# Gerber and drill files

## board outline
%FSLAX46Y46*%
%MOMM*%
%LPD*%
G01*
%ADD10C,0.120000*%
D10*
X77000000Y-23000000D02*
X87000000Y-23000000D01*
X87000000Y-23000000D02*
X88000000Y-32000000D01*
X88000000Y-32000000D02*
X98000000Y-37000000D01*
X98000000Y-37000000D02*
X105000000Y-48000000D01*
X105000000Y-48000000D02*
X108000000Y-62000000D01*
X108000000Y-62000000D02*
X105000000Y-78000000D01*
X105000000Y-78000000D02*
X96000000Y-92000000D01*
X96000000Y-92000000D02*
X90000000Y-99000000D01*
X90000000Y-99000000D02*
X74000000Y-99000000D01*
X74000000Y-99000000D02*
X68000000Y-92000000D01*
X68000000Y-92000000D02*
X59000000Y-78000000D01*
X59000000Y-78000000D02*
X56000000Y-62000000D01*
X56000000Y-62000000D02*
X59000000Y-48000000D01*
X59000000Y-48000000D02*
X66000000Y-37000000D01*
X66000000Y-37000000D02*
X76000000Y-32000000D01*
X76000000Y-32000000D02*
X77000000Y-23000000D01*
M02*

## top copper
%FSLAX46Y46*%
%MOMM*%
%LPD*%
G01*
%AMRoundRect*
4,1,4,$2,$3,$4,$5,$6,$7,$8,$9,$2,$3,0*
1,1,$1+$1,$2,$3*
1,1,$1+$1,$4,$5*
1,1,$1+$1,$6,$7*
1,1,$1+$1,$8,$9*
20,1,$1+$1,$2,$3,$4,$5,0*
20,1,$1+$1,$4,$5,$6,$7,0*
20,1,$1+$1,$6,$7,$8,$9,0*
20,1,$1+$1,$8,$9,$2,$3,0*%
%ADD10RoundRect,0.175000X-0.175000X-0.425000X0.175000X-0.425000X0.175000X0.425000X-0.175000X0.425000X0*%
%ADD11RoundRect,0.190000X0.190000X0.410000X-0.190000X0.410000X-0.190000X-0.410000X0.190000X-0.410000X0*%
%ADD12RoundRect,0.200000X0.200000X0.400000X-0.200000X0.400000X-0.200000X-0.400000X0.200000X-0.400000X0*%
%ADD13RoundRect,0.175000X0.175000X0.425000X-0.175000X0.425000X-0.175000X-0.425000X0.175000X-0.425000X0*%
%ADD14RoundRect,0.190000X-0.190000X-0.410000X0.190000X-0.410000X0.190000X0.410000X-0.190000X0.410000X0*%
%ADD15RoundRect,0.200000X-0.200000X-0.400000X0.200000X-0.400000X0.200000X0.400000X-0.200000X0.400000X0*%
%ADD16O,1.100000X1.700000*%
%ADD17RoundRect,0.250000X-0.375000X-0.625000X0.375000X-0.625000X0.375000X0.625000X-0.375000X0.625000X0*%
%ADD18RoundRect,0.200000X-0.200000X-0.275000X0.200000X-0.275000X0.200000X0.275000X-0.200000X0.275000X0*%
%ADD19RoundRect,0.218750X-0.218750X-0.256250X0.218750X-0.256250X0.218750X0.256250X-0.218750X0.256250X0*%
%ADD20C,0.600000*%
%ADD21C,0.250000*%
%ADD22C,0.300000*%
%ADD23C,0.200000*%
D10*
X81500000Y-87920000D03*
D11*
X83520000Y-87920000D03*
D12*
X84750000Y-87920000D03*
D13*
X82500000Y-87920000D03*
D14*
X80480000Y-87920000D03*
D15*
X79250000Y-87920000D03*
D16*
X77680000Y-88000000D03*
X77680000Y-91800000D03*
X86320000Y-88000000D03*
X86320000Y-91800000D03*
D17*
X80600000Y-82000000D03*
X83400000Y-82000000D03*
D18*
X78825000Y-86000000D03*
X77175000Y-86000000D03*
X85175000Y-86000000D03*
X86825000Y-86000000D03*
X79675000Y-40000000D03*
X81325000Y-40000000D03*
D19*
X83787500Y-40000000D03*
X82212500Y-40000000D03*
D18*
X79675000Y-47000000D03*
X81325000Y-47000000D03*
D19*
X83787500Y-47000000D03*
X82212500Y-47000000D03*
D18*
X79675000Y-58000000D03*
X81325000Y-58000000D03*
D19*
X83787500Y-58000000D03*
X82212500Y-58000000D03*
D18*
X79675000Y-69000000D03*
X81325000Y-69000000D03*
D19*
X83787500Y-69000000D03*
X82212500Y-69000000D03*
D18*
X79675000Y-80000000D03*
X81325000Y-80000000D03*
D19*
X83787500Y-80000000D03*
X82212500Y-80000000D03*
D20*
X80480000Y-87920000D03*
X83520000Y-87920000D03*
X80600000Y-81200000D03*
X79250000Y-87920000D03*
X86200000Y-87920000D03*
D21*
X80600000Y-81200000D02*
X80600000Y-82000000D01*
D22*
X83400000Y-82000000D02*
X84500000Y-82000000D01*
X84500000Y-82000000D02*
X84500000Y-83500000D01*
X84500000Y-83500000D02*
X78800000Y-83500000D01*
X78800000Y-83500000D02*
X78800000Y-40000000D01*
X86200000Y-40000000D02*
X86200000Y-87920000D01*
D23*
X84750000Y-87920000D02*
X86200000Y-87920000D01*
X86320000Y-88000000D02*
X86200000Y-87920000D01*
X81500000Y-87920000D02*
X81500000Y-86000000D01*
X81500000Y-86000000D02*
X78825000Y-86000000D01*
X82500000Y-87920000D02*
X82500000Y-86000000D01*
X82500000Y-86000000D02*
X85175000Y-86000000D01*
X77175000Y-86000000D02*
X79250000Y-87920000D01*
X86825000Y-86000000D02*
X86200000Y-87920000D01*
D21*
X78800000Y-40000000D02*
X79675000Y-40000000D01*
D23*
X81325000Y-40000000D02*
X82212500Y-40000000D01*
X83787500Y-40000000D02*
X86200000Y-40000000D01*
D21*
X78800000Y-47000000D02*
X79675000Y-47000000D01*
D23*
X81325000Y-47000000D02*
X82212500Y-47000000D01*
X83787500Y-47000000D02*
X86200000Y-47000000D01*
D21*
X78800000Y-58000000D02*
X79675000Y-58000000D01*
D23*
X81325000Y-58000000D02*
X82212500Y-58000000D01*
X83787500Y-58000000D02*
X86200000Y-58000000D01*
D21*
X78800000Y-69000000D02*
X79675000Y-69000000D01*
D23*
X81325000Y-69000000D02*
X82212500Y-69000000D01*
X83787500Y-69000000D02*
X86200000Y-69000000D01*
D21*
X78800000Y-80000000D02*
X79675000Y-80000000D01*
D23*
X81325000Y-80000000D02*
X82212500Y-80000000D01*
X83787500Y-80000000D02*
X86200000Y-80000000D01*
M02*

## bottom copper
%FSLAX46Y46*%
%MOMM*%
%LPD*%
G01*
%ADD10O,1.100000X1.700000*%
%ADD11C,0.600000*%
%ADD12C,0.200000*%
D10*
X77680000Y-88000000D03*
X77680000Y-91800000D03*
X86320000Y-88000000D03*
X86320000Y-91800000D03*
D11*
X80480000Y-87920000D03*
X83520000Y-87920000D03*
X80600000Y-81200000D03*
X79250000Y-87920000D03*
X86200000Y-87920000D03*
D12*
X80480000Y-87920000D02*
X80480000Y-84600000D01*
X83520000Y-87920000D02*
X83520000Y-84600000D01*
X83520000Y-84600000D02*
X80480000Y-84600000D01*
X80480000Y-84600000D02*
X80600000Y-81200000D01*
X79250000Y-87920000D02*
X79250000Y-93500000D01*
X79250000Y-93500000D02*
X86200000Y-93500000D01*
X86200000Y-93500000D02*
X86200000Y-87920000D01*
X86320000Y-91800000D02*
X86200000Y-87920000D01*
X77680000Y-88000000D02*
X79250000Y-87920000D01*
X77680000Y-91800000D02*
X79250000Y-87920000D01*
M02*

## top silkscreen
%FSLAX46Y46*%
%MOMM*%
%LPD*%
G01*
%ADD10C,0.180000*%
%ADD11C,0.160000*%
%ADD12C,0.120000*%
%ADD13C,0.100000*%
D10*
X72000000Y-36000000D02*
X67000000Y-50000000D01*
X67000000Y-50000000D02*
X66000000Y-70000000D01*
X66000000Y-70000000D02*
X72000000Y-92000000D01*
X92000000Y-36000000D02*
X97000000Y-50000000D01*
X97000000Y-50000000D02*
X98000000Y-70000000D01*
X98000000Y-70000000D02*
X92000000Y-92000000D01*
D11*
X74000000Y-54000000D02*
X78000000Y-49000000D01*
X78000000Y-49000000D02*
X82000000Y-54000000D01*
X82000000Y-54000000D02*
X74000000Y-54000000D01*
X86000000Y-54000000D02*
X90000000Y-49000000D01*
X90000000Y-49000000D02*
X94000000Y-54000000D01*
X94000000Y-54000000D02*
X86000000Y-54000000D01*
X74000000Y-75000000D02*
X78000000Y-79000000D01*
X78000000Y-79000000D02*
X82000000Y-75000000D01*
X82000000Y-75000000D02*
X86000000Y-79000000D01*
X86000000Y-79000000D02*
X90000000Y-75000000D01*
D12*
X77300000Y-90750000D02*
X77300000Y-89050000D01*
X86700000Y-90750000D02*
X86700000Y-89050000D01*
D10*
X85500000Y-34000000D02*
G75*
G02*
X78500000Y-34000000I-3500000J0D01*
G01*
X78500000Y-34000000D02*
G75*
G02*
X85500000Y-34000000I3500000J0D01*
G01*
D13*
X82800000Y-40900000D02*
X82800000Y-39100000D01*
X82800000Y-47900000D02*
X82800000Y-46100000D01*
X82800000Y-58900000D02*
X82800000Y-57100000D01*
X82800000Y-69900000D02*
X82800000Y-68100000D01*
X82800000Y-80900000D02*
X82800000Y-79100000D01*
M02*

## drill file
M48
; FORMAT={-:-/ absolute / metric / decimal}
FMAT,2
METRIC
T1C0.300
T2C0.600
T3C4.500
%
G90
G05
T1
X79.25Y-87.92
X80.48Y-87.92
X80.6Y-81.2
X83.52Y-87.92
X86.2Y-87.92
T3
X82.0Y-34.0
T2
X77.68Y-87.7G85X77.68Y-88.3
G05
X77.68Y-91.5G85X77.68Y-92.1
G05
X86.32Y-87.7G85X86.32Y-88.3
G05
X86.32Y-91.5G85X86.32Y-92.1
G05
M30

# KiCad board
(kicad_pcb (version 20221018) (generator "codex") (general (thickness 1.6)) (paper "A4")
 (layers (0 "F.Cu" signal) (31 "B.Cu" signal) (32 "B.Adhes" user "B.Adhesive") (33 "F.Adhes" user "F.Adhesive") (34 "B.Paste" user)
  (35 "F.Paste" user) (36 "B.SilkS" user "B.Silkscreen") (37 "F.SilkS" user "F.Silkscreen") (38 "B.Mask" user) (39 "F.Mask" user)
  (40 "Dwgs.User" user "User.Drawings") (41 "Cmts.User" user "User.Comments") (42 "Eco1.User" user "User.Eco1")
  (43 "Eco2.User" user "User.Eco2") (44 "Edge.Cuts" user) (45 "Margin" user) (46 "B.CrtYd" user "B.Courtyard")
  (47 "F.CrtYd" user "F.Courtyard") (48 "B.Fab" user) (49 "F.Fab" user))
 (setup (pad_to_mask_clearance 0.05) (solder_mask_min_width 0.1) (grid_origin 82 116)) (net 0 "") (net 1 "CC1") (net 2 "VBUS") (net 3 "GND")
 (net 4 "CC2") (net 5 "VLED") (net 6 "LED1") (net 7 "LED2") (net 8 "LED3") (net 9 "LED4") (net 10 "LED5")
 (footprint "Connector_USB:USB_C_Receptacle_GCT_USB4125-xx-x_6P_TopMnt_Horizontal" (layer "F.Cu") (at 82 91)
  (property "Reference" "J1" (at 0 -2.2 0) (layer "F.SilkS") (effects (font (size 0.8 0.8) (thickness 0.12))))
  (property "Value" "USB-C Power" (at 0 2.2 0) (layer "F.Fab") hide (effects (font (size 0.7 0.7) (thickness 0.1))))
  (fp_line (start -4.7 -0.25) (end -4.7 -1.95) (stroke (width 0.12) (type solid)) (layer "F.SilkS"))
  (fp_line (start 4.7 -0.25) (end 4.7 -1.95) (stroke (width 0.12) (type solid)) (layer "F.SilkS"))
  (pad "A5" smd roundrect (at -0.5 -3.08) (size 0.7 1.2) (layers "F.Cu" "F.Paste" "F.Mask") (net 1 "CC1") (roundrect_rratio 0.25))
  (pad "A9" smd roundrect (at 1.52 -3.08 180) (size 0.76 1.2) (layers "F.Cu" "F.Paste" "F.Mask") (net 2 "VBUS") (roundrect_rratio 0.25))
  (pad "A12" smd roundrect (at 2.75 -3.08 180) (size 0.8 1.2) (layers "F.Cu" "F.Paste" "F.Mask") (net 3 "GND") (roundrect_rratio 0.25))
  (pad "B5" smd roundrect (at 0.5 -3.08 180) (size 0.7 1.2) (layers "F.Cu" "F.Paste" "F.Mask") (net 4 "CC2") (roundrect_rratio 0.25))
  (pad "B9" smd roundrect (at -1.52 -3.08) (size 0.76 1.2) (layers "F.Cu" "F.Paste" "F.Mask") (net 2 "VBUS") (roundrect_rratio 0.25))
  (pad "B12" smd roundrect (at -2.75 -3.08) (size 0.8 1.2) (layers "F.Cu" "F.Paste" "F.Mask") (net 3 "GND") (roundrect_rratio 0.25))
  (pad "SH" thru_hole oval (at -4.32 -3) (size 1.1 1.7) (drill oval 0.6 1.2) (layers "*.Cu" "*.Mask") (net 3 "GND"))
  (pad "SH" thru_hole oval (at -4.32 0.8) (size 1.1 1.7) (drill oval 0.6 1.2) (layers "*.Cu" "*.Mask") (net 3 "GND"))
  (pad "SH" thru_hole oval (at 4.32 -3) (size 1.1 1.7) (drill oval 0.6 1.2) (layers "*.Cu" "*.Mask") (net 3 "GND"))
  (pad "SH" thru_hole oval (at 4.32 0.8) (size 1.1 1.7) (drill oval 0.6 1.2) (layers "*.Cu" "*.Mask") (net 3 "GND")))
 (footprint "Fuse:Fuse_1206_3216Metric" (layer "F.Cu") (at 82 82)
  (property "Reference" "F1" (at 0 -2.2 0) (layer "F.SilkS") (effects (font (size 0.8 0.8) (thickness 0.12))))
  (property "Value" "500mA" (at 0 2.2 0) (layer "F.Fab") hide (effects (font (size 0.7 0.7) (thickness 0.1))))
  (pad "1" smd roundrect (at -1.4 0) (size 1.25 1.75) (layers "F.Cu" "F.Paste" "F.Mask") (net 2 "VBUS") (roundrect_rratio 0.2))
  (pad "2" smd roundrect (at 1.4 0) (size 1.25 1.75) (layers "F.Cu" "F.Paste" "F.Mask") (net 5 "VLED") (roundrect_rratio 0.2)))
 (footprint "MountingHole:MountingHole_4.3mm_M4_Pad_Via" (layer "F.Cu") (at 82 34)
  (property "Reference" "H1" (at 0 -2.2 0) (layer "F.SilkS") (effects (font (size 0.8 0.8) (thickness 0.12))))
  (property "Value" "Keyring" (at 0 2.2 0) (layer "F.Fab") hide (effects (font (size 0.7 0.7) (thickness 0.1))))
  (fp_circle (center 0 0) (end 3.5 0) (stroke (width 0.18) (type solid)) (fill none) (layer "F.SilkS"))
  (pad "1" np_thru_hole circle (at 0 0) (size 4.5 4.5) (drill 4.5) (layers "*.Cu" "*.Mask")))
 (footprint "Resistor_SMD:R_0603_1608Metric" (layer "F.Cu") (at 78 86 180)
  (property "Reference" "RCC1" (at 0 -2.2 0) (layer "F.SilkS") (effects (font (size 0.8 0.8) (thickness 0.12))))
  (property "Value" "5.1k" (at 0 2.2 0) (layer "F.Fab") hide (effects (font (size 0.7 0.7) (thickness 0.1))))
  (pad "1" smd roundrect (at -0.825 0) (size 0.8 0.95) (layers "F.Cu" "F.Paste" "F.Mask") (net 1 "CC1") (roundrect_rratio 0.25))
  (pad "2" smd roundrect (at 0.825 0) (size 0.8 0.95) (layers "F.Cu" "F.Paste" "F.Mask") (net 3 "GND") (roundrect_rratio 0.25)))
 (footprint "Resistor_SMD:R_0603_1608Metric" (layer "F.Cu") (at 86 86)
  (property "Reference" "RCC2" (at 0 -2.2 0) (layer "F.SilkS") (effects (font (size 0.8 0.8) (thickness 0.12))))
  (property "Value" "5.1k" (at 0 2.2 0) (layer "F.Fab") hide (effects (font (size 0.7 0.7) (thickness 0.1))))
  (pad "1" smd roundrect (at -0.825 0) (size 0.8 0.95) (layers "F.Cu" "F.Paste" "F.Mask") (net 4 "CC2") (roundrect_rratio 0.25))
  (pad "2" smd roundrect (at 0.825 0) (size 0.8 0.95) (layers "F.Cu" "F.Paste" "F.Mask") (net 3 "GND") (roundrect_rratio 0.25)))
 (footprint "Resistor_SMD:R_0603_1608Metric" (layer "F.Cu") (at 80.5 40 0)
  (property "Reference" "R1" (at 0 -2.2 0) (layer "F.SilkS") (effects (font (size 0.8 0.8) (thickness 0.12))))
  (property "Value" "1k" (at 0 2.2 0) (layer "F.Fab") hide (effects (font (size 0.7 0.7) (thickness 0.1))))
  (pad "1" smd roundrect (at -0.825 0) (size 0.8 0.95) (layers "F.Cu" "F.Paste" "F.Mask") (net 5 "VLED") (roundrect_rratio 0.25))
  (pad "2" smd roundrect (at 0.825 0) (size 0.8 0.95) (layers "F.Cu" "F.Paste" "F.Mask") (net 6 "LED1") (roundrect_rratio 0.25)))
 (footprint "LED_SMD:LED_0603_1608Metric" (layer "F.Cu") (at 83 40 180)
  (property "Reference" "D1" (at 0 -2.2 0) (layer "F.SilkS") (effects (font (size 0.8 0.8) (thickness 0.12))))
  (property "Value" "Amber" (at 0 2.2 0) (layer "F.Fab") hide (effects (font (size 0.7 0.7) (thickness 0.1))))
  (fp_line (start 0.2 -0.9) (end 0.2 0.9) (stroke (width 0.1) (type solid)) (layer "F.SilkS"))
  (pad "1" smd roundrect (at -0.7875 0) (size 0.875 0.95) (layers "F.Cu" "F.Paste" "F.Mask") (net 3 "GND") (roundrect_rratio 0.25))
  (pad "2" smd roundrect (at 0.7875 0) (size 0.875 0.95) (layers "F.Cu" "F.Paste" "F.Mask") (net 6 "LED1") (roundrect_rratio 0.25)))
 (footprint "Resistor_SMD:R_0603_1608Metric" (layer "F.Cu") (at 80.5 47 0)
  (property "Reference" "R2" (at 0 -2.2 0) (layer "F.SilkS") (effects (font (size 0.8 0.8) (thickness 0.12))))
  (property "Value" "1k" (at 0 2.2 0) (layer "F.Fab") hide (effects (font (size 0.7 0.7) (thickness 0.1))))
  (pad "1" smd roundrect (at -0.825 0) (size 0.8 0.95) (layers "F.Cu" "F.Paste" "F.Mask") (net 5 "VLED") (roundrect_rratio 0.25))
  (pad "2" smd roundrect (at 0.825 0) (size 0.8 0.95) (layers "F.Cu" "F.Paste" "F.Mask") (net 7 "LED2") (roundrect_rratio 0.25)))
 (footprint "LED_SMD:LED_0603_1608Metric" (layer "F.Cu") (at 83 47 180)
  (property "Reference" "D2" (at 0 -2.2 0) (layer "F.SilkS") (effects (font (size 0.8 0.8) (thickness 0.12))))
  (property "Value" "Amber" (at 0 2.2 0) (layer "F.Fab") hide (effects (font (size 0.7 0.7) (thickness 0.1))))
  (fp_line (start 0.2 -0.9) (end 0.2 0.9) (stroke (width 0.1) (type solid)) (layer "F.SilkS"))
  (pad "1" smd roundrect (at -0.7875 0) (size 0.875 0.95) (layers "F.Cu" "F.Paste" "F.Mask") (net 3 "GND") (roundrect_rratio 0.25))
  (pad "2" smd roundrect (at 0.7875 0) (size 0.875 0.95) (layers "F.Cu" "F.Paste" "F.Mask") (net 7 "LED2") (roundrect_rratio 0.25)))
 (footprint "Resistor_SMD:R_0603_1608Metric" (layer "F.Cu") (at 80.5 58 0)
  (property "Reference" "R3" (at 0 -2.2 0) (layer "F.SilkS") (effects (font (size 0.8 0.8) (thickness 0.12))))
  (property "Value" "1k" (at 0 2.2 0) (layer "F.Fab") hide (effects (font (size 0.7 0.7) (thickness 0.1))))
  (pad "1" smd roundrect (at -0.825 0) (size 0.8 0.95) (layers "F.Cu" "F.Paste" "F.Mask") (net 5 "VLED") (roundrect_rratio 0.25))
  (pad "2" smd roundrect (at 0.825 0) (size 0.8 0.95) (layers "F.Cu" "F.Paste" "F.Mask") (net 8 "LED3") (roundrect_rratio 0.25)))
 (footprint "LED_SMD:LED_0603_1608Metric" (layer "F.Cu") (at 83 58 180)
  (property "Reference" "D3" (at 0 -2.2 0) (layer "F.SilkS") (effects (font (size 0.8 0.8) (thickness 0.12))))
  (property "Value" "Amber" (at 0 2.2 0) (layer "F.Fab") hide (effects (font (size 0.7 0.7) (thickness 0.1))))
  (fp_line (start 0.2 -0.9) (end 0.2 0.9) (stroke (width 0.1) (type solid)) (layer "F.SilkS"))
  (pad "1" smd roundrect (at -0.7875 0) (size 0.875 0.95) (layers "F.Cu" "F.Paste" "F.Mask") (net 3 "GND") (roundrect_rratio 0.25))
  (pad "2" smd roundrect (at 0.7875 0) (size 0.875 0.95) (layers "F.Cu" "F.Paste" "F.Mask") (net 8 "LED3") (roundrect_rratio 0.25)))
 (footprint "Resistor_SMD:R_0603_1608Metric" (layer "F.Cu") (at 80.5 69 0)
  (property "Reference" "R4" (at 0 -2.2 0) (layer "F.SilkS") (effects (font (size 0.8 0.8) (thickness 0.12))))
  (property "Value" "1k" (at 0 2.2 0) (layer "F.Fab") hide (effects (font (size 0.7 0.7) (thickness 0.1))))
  (pad "1" smd roundrect (at -0.825 0) (size 0.8 0.95) (layers "F.Cu" "F.Paste" "F.Mask") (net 5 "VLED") (roundrect_rratio 0.25))
  (pad "2" smd roundrect (at 0.825 0) (size 0.8 0.95) (layers "F.Cu" "F.Paste" "F.Mask") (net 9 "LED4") (roundrect_rratio 0.25)))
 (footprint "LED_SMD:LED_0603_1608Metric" (layer "F.Cu") (at 83 69 180)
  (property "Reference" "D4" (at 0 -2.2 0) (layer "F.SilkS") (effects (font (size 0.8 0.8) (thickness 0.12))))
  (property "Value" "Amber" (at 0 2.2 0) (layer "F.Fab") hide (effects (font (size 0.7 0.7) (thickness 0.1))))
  (fp_line (start 0.2 -0.9) (end 0.2 0.9) (stroke (width 0.1) (type solid)) (layer "F.SilkS"))
  (pad "1" smd roundrect (at -0.7875 0) (size 0.875 0.95) (layers "F.Cu" "F.Paste" "F.Mask") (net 3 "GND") (roundrect_rratio 0.25))
  (pad "2" smd roundrect (at 0.7875 0) (size 0.875 0.95) (layers "F.Cu" "F.Paste" "F.Mask") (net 9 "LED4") (roundrect_rratio 0.25)))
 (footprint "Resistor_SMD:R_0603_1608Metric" (layer "F.Cu") (at 80.5 80 0)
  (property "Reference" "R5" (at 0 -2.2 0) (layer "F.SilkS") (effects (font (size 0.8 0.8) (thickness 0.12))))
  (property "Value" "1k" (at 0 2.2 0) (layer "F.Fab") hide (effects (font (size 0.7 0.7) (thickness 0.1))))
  (pad "1" smd roundrect (at -0.825 0) (size 0.8 0.95) (layers "F.Cu" "F.Paste" "F.Mask") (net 5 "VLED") (roundrect_rratio 0.25))
  (pad "2" smd roundrect (at 0.825 0) (size 0.8 0.95) (layers "F.Cu" "F.Paste" "F.Mask") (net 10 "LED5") (roundrect_rratio 0.25)))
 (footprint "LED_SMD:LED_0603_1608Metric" (layer "F.Cu") (at 83 80 180)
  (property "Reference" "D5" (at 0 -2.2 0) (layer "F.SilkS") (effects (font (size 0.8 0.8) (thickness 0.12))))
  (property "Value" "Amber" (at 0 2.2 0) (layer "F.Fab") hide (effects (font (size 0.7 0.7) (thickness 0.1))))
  (fp_line (start 0.2 -0.9) (end 0.2 0.9) (stroke (width 0.1) (type solid)) (layer "F.SilkS"))
  (pad "1" smd roundrect (at -0.7875 0) (size 0.875 0.95) (layers "F.Cu" "F.Paste" "F.Mask") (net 3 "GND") (roundrect_rratio 0.25))
  (pad "2" smd roundrect (at 0.7875 0) (size 0.875 0.95) (layers "F.Cu" "F.Paste" "F.Mask") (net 10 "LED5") (roundrect_rratio 0.25)))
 (gr_line (start 77 23) (end 87 23) (stroke (width 0.12) (type solid)) (layer "Edge.Cuts"))
 (gr_line (start 87 23) (end 88 32) (stroke (width 0.12) (type solid)) (layer "Edge.Cuts"))
 (gr_line (start 88 32) (end 98 37) (stroke (width 0.12) (type solid)) (layer "Edge.Cuts"))
 (gr_line (start 98 37) (end 105 48) (stroke (width 0.12) (type solid)) (layer "Edge.Cuts"))
 (gr_line (start 105 48) (end 108 62) (stroke (width 0.12) (type solid)) (layer "Edge.Cuts"))
 (gr_line (start 108 62) (end 105 78) (stroke (width 0.12) (type solid)) (layer "Edge.Cuts"))
 (gr_line (start 105 78) (end 96 92) (stroke (width 0.12) (type solid)) (layer "Edge.Cuts"))
 (gr_line (start 96 92) (end 90 99) (stroke (width 0.12) (type solid)) (layer "Edge.Cuts"))
 (gr_line (start 90 99) (end 74 99) (stroke (width 0.12) (type solid)) (layer "Edge.Cuts"))
 (gr_line (start 74 99) (end 68 92) (stroke (width 0.12) (type solid)) (layer "Edge.Cuts"))
 (gr_line (start 68 92) (end 59 78) (stroke (width 0.12) (type solid)) (layer "Edge.Cuts"))
 (gr_line (start 59 78) (end 56 62) (stroke (width 0.12) (type solid)) (layer "Edge.Cuts"))
 (gr_line (start 56 62) (end 59 48) (stroke (width 0.12) (type solid)) (layer "Edge.Cuts"))
 (gr_line (start 59 48) (end 66 37) (stroke (width 0.12) (type solid)) (layer "Edge.Cuts"))
 (gr_line (start 66 37) (end 76 32) (stroke (width 0.12) (type solid)) (layer "Edge.Cuts"))
 (gr_line (start 76 32) (end 77 23) (stroke (width 0.12) (type solid)) (layer "Edge.Cuts"))
 (gr_line (start 72 36) (end 67 50) (stroke (width 0.18) (type solid)) (layer "F.SilkS"))
 (gr_line (start 67 50) (end 66 70) (stroke (width 0.18) (type solid)) (layer "F.SilkS"))
 (gr_line (start 66 70) (end 72 92) (stroke (width 0.18) (type solid)) (layer "F.SilkS"))
 (gr_line (start 92 36) (end 97 50) (stroke (width 0.18) (type solid)) (layer "F.SilkS"))
 (gr_line (start 97 50) (end 98 70) (stroke (width 0.18) (type solid)) (layer "F.SilkS"))
 (gr_line (start 98 70) (end 92 92) (stroke (width 0.18) (type solid)) (layer "F.SilkS"))
 (gr_line (start 74 54) (end 78 49) (stroke (width 0.16) (type solid)) (layer "F.SilkS"))
 (gr_line (start 78 49) (end 82 54) (stroke (width 0.16) (type solid)) (layer "F.SilkS"))
 (gr_line (start 82 54) (end 74 54) (stroke (width 0.16) (type solid)) (layer "F.SilkS"))
 (gr_line (start 86 54) (end 90 49) (stroke (width 0.16) (type solid)) (layer "F.SilkS"))
 (gr_line (start 90 49) (end 94 54) (stroke (width 0.16) (type solid)) (layer "F.SilkS"))
 (gr_line (start 94 54) (end 86 54) (stroke (width 0.16) (type solid)) (layer "F.SilkS"))
 (gr_line (start 74 75) (end 78 79) (stroke (width 0.16) (type solid)) (layer "F.SilkS"))
 (gr_line (start 78 79) (end 82 75) (stroke (width 0.16) (type solid)) (layer "F.SilkS"))
 (gr_line (start 82 75) (end 86 79) (stroke (width 0.16) (type solid)) (layer "F.SilkS"))
 (gr_line (start 86 79) (end 90 75) (stroke (width 0.16) (type solid)) (layer "F.SilkS"))
 (via (at 80.48 87.92) (size 0.6) (drill 0.3) (layers "F.Cu" "B.Cu") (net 2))
 (via (at 83.52 87.92) (size 0.6) (drill 0.3) (layers "F.Cu" "B.Cu") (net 2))
 (via (at 80.6 81.2) (size 0.6) (drill 0.3) (layers "F.Cu" "B.Cu") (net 2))
 (via (at 79.25 87.92) (size 0.6) (drill 0.3) (layers "F.Cu" "B.Cu") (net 3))
 (via (at 86.2 87.92) (size 0.6) (drill 0.3) (layers "F.Cu" "B.Cu") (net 3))
 (segment (start 80.6 81.2) (end 80.6 82.0) (width 0.25) (layer "F.Cu") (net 2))
 (segment (start 80.48 87.92) (end 80.48 84.6) (width 0.20) (layer "B.Cu") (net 2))
 (segment (start 83.52 87.92) (end 83.52 84.6) (width 0.20) (layer "B.Cu") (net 2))
 (segment (start 83.52 84.6) (end 80.48 84.6) (width 0.20) (layer "B.Cu") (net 2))
 (segment (start 80.48 84.6) (end 80.6 81.2) (width 0.20) (layer "B.Cu") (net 2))
 (segment (start 83.4 82.0) (end 84.5 82.0) (width 0.30) (layer "F.Cu") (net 5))
 (segment (start 84.5 82.0) (end 84.5 83.5) (width 0.30) (layer "F.Cu") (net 5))
 (segment (start 84.5 83.5) (end 78.8 83.5) (width 0.30) (layer "F.Cu") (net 5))
 (segment (start 78.8 83.5) (end 78.8 40.0) (width 0.30) (layer "F.Cu") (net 5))
 (segment (start 86.2 40.0) (end 86.2 87.92) (width 0.30) (layer "F.Cu") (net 3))
 (segment (start 84.75 87.92) (end 86.2 87.92) (width 0.20) (layer "F.Cu") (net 3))
 (segment (start 79.25 87.92) (end 79.25 93.5) (width 0.20) (layer "B.Cu") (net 3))
 (segment (start 79.25 93.5) (end 86.2 93.5) (width 0.20) (layer "B.Cu") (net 3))
 (segment (start 86.2 93.5) (end 86.2 87.92) (width 0.20) (layer "B.Cu") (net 3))
 (segment (start 86.32 88.0) (end 86.2 87.92) (width 0.20) (layer "F.Cu") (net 3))
 (segment (start 86.32 91.8) (end 86.2 87.92) (width 0.20) (layer "B.Cu") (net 3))
 (segment (start 77.68 88.0) (end 79.25 87.92) (width 0.20) (layer "B.Cu") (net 3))
 (segment (start 77.68 91.8) (end 79.25 87.92) (width 0.20) (layer "B.Cu") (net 3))
 (segment (start 81.5 87.92) (end 81.5 86.0) (width 0.20) (layer "F.Cu") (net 1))
 (segment (start 81.5 86.0) (end 78.825 86.0) (width 0.20) (layer "F.Cu") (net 1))
 (segment (start 82.5 87.92) (end 82.5 86.0) (width 0.20) (layer "F.Cu") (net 4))
 (segment (start 82.5 86.0) (end 85.175 86.0) (width 0.20) (layer "F.Cu") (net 4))
 (segment (start 77.175 86.0) (end 79.25 87.92) (width 0.20) (layer "F.Cu") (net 3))
 (segment (start 86.825 86.0) (end 86.2 87.92) (width 0.20) (layer "F.Cu") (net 3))
 (segment (start 78.8 40.0) (end 79.675 40.0) (width 0.25) (layer "F.Cu") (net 5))
 (segment (start 81.325 40.0) (end 82.2125 40.0) (width 0.20) (layer "F.Cu") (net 6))
 (segment (start 83.7875 40.0) (end 86.2 40.0) (width 0.20) (layer "F.Cu") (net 3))
 (segment (start 78.8 47.0) (end 79.675 47.0) (width 0.25) (layer "F.Cu") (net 5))
 (segment (start 81.325 47.0) (end 82.2125 47.0) (width 0.20) (layer "F.Cu") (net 7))
 (segment (start 83.7875 47.0) (end 86.2 47.0) (width 0.20) (layer "F.Cu") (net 3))
 (segment (start 78.8 58.0) (end 79.675 58.0) (width 0.25) (layer "F.Cu") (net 5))
 (segment (start 81.325 58.0) (end 82.2125 58.0) (width 0.20) (layer "F.Cu") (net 8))
 (segment (start 83.7875 58.0) (end 86.2 58.0) (width 0.20) (layer "F.Cu") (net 3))
 (segment (start 78.8 69.0) (end 79.675 69.0) (width 0.25) (layer "F.Cu") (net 5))
 (segment (start 81.325 69.0) (end 82.2125 69.0) (width 0.20) (layer "F.Cu") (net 9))
 (segment (start 83.7875 69.0) (end 86.2 69.0) (width 0.20) (layer "F.Cu") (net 3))
 (segment (start 78.8 80.0) (end 79.675 80.0) (width 0.25) (layer "F.Cu") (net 5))
 (segment (start 81.325 80.0) (end 82.2125 80.0) (width 0.20) (layer "F.Cu") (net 10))
 (segment (start 83.7875 80.0) (end 86.2 80.0) (width 0.20) (layer "F.Cu") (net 3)))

